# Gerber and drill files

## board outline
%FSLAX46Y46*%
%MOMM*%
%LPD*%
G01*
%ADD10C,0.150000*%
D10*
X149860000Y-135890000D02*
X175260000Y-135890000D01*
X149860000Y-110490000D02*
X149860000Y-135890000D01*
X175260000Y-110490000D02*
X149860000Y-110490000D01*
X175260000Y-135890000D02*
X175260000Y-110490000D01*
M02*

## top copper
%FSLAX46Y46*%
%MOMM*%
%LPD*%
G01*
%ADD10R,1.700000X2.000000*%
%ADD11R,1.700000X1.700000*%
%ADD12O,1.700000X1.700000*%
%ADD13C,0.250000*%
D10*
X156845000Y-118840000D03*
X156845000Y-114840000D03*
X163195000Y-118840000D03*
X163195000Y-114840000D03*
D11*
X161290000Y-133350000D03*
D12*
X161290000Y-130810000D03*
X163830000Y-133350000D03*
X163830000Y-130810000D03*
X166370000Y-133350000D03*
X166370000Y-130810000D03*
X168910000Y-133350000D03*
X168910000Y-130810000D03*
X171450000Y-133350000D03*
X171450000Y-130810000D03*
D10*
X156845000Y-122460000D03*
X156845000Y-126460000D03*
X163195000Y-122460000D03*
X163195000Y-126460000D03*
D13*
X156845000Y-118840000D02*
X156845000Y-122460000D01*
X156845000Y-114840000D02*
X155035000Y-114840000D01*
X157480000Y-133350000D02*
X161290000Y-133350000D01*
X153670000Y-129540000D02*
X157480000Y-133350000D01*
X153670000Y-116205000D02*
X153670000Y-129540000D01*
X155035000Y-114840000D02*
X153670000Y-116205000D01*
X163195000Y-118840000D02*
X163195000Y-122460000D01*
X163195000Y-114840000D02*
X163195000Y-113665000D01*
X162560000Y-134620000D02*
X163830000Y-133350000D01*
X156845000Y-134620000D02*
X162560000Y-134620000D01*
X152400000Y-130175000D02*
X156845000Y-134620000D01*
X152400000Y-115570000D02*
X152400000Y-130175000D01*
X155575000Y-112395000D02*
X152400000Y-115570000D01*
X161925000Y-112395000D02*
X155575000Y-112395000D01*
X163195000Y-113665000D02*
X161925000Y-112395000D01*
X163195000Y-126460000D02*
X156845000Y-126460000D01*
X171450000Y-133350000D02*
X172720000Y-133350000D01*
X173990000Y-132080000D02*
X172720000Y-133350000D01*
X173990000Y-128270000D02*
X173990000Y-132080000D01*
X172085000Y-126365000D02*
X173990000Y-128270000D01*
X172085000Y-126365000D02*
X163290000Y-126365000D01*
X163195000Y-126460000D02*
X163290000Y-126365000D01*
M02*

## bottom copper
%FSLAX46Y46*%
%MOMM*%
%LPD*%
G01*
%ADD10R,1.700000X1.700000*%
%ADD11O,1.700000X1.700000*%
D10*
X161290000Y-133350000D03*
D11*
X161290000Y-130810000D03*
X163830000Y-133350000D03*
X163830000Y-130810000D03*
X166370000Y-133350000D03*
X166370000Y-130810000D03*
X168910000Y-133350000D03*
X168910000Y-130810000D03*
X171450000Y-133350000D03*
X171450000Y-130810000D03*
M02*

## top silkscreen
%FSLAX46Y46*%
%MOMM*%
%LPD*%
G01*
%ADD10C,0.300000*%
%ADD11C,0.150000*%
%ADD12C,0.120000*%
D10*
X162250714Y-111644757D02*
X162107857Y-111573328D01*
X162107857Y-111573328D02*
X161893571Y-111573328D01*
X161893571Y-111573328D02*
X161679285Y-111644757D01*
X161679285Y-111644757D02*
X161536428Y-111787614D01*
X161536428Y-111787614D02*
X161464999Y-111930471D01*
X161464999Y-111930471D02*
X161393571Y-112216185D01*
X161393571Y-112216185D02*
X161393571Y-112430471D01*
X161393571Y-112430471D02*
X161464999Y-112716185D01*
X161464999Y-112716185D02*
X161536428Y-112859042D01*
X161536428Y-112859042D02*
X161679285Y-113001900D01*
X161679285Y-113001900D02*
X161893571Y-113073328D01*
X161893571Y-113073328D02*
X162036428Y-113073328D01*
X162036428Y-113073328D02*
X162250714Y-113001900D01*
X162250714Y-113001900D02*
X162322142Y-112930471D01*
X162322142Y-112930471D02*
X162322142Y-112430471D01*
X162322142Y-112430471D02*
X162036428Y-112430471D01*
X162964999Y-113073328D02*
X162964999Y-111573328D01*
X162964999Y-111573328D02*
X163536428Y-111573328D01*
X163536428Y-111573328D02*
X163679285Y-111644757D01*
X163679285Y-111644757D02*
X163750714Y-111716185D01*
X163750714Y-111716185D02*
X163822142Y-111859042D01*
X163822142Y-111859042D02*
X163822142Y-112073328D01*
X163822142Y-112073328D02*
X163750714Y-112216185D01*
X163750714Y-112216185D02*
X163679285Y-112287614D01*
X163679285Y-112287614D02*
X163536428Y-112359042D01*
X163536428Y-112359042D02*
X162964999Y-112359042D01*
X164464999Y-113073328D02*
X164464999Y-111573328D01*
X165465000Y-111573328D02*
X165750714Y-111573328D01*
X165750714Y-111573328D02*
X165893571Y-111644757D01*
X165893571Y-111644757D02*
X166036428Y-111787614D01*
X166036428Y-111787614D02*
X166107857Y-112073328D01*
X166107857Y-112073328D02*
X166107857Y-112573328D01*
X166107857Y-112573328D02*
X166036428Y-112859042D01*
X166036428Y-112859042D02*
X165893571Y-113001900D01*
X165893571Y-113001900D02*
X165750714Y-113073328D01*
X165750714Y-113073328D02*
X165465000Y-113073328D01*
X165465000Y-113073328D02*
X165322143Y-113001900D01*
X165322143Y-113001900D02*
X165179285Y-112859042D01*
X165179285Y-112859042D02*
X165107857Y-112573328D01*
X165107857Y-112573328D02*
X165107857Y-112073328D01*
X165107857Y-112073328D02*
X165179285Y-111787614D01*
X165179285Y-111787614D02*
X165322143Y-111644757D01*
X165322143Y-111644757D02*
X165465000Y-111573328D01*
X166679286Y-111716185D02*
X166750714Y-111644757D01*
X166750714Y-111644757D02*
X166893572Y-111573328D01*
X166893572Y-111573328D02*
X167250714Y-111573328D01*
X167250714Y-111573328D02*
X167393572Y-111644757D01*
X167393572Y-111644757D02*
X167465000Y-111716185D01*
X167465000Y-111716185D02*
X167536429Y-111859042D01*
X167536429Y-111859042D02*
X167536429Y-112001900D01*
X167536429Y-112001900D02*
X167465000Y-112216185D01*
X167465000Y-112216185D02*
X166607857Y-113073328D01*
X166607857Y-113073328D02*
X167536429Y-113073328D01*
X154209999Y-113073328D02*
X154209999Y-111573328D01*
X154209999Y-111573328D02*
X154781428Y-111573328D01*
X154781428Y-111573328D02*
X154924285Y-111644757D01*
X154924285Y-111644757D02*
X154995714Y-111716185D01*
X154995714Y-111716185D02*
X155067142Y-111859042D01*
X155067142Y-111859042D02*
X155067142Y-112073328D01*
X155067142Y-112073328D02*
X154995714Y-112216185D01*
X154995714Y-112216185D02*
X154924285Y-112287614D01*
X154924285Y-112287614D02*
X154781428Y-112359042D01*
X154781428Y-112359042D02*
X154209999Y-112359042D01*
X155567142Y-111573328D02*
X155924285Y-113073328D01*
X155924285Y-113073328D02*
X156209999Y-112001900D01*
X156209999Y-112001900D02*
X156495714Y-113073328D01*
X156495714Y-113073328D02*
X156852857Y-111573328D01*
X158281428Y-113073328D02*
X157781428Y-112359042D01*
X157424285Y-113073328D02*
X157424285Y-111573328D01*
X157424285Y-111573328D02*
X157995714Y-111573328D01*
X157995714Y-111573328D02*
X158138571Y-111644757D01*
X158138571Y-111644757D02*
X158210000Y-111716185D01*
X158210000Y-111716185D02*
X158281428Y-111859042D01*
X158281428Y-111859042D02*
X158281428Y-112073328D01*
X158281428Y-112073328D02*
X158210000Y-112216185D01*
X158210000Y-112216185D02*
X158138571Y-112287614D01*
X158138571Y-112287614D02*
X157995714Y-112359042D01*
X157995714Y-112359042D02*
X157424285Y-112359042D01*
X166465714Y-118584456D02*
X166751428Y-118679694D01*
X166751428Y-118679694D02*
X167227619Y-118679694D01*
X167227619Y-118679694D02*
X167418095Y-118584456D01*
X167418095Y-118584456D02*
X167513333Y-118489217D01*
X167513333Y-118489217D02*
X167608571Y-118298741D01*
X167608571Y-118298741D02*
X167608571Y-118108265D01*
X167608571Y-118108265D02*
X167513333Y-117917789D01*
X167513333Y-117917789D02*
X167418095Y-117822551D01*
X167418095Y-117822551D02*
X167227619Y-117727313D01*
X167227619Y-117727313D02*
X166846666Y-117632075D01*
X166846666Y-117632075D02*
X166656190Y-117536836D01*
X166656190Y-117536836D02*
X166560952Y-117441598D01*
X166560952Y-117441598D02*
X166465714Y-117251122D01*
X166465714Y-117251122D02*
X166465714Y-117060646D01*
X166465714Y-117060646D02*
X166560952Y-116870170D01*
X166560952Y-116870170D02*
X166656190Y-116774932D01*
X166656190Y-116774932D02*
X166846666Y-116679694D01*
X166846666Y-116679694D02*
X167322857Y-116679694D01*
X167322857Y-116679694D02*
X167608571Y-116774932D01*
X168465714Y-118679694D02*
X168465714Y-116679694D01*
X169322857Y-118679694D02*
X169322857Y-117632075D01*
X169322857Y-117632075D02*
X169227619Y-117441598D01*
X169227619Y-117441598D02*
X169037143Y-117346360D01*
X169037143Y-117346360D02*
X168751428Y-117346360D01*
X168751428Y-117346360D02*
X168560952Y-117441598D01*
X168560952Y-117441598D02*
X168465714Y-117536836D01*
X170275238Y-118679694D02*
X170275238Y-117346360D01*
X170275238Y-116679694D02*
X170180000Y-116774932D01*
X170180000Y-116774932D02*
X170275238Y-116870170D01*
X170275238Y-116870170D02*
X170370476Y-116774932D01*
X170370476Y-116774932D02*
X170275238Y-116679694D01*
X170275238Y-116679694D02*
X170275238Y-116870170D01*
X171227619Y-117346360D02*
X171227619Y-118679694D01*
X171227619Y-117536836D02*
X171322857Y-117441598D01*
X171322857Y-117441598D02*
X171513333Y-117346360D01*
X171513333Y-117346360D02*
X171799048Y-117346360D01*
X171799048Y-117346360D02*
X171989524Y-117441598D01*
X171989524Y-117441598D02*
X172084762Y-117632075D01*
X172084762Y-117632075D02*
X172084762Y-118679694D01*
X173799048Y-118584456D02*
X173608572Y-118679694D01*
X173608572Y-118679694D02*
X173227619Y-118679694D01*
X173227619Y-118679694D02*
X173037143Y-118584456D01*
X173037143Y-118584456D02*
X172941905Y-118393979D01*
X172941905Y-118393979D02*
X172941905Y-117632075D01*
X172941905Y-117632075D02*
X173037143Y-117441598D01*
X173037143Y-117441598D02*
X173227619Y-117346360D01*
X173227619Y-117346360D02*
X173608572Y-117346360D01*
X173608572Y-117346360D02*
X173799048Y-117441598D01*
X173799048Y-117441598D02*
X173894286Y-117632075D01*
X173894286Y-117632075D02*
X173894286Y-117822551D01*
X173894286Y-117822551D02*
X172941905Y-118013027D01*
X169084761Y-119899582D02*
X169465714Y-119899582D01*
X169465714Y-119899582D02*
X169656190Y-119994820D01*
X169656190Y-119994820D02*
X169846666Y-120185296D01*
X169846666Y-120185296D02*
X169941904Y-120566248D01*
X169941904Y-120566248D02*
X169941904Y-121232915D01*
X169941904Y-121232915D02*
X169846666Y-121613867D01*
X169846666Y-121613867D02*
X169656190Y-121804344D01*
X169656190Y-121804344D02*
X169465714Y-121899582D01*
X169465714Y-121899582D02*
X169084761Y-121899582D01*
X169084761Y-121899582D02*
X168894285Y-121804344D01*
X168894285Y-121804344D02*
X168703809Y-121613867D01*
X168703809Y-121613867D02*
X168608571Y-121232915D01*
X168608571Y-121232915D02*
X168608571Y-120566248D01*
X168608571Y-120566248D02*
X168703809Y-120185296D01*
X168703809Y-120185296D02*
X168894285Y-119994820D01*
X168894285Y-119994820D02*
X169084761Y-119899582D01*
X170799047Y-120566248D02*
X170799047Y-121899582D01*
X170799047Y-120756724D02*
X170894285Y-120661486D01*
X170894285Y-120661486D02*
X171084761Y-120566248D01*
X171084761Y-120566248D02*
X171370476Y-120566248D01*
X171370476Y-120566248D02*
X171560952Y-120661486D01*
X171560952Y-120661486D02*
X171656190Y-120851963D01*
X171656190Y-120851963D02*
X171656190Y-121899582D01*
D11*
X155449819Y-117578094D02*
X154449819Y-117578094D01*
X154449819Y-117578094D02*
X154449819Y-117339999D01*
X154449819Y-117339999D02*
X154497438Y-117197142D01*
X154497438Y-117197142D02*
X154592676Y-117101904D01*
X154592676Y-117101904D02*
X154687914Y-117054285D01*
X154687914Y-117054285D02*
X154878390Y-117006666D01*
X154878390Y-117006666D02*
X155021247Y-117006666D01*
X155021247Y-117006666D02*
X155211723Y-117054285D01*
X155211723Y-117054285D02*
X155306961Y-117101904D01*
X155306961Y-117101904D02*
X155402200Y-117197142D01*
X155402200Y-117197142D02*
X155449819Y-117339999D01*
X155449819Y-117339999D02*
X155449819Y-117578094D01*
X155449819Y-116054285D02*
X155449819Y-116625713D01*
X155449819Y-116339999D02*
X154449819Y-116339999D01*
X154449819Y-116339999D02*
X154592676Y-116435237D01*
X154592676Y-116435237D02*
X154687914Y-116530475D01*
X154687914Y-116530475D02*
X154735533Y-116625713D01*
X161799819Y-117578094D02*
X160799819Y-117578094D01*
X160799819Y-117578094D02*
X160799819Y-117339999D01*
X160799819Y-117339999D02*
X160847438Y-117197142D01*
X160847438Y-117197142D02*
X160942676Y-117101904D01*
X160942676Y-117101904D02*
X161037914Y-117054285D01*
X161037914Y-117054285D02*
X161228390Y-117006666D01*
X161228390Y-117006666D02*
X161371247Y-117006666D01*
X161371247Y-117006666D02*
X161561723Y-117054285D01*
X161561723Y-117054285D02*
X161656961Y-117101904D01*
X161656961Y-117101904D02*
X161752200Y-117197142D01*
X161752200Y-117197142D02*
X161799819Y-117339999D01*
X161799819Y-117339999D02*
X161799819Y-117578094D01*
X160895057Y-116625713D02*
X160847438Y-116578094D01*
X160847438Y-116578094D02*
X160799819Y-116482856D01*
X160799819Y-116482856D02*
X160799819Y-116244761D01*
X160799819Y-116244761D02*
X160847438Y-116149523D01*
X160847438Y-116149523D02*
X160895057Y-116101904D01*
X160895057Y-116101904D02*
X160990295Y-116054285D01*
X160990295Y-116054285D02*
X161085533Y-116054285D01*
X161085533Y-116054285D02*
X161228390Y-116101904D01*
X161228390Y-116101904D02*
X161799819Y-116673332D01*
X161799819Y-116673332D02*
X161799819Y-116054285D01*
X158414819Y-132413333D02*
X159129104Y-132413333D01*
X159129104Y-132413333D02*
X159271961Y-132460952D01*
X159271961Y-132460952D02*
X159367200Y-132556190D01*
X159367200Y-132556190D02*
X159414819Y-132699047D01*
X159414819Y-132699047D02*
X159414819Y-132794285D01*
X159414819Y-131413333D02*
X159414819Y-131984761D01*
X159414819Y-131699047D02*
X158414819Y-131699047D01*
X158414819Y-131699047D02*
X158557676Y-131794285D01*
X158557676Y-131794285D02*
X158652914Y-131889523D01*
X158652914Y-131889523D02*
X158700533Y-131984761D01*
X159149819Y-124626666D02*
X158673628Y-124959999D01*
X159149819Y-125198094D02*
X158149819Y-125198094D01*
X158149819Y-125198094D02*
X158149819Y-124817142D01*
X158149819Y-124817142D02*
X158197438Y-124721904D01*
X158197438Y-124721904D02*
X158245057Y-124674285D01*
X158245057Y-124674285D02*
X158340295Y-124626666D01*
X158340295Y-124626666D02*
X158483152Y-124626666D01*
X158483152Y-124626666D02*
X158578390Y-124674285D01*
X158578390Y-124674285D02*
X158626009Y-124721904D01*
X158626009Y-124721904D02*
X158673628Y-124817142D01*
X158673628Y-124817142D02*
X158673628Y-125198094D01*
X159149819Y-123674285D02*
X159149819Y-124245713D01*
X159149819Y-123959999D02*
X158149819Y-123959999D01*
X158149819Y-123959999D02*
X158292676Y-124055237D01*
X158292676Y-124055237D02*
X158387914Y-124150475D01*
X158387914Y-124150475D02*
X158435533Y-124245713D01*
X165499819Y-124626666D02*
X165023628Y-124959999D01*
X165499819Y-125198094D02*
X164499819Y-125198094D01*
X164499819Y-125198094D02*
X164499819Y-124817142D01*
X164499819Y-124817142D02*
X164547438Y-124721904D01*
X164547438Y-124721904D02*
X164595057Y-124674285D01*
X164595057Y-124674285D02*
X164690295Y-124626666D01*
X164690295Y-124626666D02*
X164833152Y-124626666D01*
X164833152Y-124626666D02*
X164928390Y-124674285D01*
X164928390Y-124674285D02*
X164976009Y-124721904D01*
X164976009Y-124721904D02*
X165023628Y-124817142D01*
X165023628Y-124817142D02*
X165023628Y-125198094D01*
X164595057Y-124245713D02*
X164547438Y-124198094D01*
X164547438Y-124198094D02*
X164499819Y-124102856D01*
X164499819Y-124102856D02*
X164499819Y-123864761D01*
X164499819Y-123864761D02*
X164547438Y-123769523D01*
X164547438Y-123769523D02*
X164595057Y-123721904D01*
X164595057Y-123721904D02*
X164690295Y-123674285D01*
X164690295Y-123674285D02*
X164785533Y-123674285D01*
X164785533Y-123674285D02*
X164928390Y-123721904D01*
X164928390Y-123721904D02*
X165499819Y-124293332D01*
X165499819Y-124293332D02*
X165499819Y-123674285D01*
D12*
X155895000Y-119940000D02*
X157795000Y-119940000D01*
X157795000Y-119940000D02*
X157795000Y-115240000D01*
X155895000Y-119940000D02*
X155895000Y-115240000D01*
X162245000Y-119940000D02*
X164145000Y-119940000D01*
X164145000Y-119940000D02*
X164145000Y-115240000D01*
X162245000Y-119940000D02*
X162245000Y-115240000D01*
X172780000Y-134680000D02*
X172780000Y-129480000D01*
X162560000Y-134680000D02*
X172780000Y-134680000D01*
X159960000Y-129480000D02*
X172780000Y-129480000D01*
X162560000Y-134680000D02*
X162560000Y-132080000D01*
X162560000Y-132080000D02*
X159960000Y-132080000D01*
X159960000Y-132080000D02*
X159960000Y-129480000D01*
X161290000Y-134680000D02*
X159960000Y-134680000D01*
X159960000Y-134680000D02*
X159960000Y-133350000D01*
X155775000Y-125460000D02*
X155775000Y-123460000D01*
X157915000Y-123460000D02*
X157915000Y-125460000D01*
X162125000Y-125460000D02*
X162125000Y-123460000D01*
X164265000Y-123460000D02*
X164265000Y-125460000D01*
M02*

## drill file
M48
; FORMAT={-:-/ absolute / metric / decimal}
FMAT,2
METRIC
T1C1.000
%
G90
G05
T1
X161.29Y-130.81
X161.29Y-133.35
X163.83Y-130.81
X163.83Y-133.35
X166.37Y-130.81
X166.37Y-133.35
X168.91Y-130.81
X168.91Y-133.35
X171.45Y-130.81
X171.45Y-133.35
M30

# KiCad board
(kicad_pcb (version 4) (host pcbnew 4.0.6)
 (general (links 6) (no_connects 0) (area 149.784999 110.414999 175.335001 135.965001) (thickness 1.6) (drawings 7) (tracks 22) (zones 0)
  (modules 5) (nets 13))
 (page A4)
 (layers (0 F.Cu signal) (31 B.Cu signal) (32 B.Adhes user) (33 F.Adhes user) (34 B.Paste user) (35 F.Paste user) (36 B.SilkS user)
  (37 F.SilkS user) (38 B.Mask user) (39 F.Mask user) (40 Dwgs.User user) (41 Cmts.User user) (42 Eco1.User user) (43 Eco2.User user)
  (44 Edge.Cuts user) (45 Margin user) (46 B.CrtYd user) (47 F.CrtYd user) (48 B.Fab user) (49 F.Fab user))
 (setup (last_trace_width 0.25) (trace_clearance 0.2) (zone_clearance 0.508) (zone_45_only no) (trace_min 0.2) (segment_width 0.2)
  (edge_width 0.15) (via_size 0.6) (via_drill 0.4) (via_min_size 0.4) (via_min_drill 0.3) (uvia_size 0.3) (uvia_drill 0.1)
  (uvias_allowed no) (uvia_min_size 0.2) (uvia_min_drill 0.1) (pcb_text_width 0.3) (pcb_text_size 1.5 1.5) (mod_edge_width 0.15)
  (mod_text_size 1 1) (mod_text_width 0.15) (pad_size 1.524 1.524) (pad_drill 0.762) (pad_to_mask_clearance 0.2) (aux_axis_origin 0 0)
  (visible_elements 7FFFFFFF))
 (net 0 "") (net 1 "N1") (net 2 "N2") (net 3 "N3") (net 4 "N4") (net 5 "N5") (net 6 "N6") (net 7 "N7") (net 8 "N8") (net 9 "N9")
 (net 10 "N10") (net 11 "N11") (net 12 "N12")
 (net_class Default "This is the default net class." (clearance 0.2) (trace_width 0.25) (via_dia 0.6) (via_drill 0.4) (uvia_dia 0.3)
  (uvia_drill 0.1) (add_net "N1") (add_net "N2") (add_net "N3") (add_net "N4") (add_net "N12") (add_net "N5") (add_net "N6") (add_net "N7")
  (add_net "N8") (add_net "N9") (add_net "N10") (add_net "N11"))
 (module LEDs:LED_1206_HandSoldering (layer F.Cu) (at 156.845 116.84 90)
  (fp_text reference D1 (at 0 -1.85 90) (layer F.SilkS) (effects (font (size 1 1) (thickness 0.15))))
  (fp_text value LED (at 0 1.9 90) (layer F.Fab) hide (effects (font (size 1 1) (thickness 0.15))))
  (fp_line (start -3.1 -0.95) (end -3.1 0.95) (layer F.SilkS) (width 0.12))
  (fp_line (start -3.1 0.95) (end 1.6 0.95) (layer F.SilkS) (width 0.12))
  (fp_line (start -3.1 -0.95) (end 1.6 -0.95) (layer F.SilkS) (width 0.12))
  (pad 1 smd rect (at -2 0 90) (size 2 1.7) (layers F.Cu F.Paste F.Mask) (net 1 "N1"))
  (pad 2 smd rect (at 2 0 90) (size 2 1.7) (layers F.Cu F.Paste F.Mask) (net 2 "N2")))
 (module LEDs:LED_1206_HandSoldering (layer F.Cu) (at 163.195 116.84 90)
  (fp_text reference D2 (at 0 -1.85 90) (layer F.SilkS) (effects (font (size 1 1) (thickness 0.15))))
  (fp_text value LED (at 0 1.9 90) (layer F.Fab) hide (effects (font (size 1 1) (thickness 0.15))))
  (fp_line (start -3.1 -0.95) (end -3.1 0.95) (layer F.SilkS) (width 0.12))
  (fp_line (start -3.1 0.95) (end 1.6 0.95) (layer F.SilkS) (width 0.12))
  (fp_line (start -3.1 -0.95) (end 1.6 -0.95) (layer F.SilkS) (width 0.12))
  (pad 1 smd rect (at -2 0 90) (size 2 1.7) (layers F.Cu F.Paste F.Mask) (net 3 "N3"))
  (pad 2 smd rect (at 2 0 90) (size 2 1.7) (layers F.Cu F.Paste F.Mask) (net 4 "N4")))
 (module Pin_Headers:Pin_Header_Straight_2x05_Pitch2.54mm (layer F.Cu) (at 161.29 133.35 90)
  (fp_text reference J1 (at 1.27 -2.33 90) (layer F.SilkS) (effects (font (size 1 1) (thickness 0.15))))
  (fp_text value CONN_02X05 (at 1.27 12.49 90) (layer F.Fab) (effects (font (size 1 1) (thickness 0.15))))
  (fp_line (start -1.33 11.49) (end 3.87 11.49) (layer F.SilkS) (width 0.12))
  (fp_line (start -1.33 1.27) (end -1.33 11.49) (layer F.SilkS) (width 0.12))
  (fp_line (start 3.87 -1.33) (end 3.87 11.49) (layer F.SilkS) (width 0.12))
  (fp_line (start -1.33 1.27) (end 1.27 1.27) (layer F.SilkS) (width 0.12))
  (fp_line (start 1.27 1.27) (end 1.27 -1.33) (layer F.SilkS) (width 0.12))
  (fp_line (start 1.27 -1.33) (end 3.87 -1.33) (layer F.SilkS) (width 0.12))
  (fp_line (start -1.33 0) (end -1.33 -1.33) (layer F.SilkS) (width 0.12))
  (fp_line (start -1.33 -1.33) (end 0 -1.33) (layer F.SilkS) (width 0.12))
  (pad 1 thru_hole rect (at 0 0 90) (size 1.7 1.7) (drill 1) (layers *.Cu *.Mask) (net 2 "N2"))
  (pad 2 thru_hole oval (at 2.54 0 90) (size 1.7 1.7) (drill 1) (layers *.Cu *.Mask) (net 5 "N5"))
  (pad 3 thru_hole oval (at 0 2.54 90) (size 1.7 1.7) (drill 1) (layers *.Cu *.Mask) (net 4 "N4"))
  (pad 4 thru_hole oval (at 2.54 2.54 90) (size 1.7 1.7) (drill 1) (layers *.Cu *.Mask) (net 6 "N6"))
  (pad 5 thru_hole oval (at 0 5.08 90) (size 1.7 1.7) (drill 1) (layers *.Cu *.Mask) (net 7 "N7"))
  (pad 6 thru_hole oval (at 2.54 5.08 90) (size 1.7 1.7) (drill 1) (layers *.Cu *.Mask) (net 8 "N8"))
  (pad 7 thru_hole oval (at 0 7.62 90) (size 1.7 1.7) (drill 1) (layers *.Cu *.Mask) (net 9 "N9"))
  (pad 8 thru_hole oval (at 2.54 7.62 90) (size 1.7 1.7) (drill 1) (layers *.Cu *.Mask) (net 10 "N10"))
  (pad 9 thru_hole oval (at 0 10.16 90) (size 1.7 1.7) (drill 1) (layers *.Cu *.Mask) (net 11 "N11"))
  (pad 10 thru_hole oval (at 2.54 10.16 90) (size 1.7 1.7) (drill 1) (layers *.Cu *.Mask) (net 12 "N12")))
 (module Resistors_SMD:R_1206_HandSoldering (layer F.Cu) (at 156.845 124.46 270)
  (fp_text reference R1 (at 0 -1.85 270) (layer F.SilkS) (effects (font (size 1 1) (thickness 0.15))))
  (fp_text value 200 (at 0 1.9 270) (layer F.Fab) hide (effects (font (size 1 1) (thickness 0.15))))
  (fp_line (start 1 1.07) (end -1 1.07) (layer F.SilkS) (width 0.12))
  (fp_line (start -1 -1.07) (end 1 -1.07) (layer F.SilkS) (width 0.12))
  (pad 1 smd rect (at -2 0 270) (size 2 1.7) (layers F.Cu F.Paste F.Mask) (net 1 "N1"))
  (pad 2 smd rect (at 2 0 270) (size 2 1.7) (layers F.Cu F.Paste F.Mask) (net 11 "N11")))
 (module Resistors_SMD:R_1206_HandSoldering (layer F.Cu) (at 163.195 124.46 270)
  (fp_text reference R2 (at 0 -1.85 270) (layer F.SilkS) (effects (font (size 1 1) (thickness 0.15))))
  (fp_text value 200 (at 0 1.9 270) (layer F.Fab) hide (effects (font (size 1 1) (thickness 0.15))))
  (fp_line (start 1 1.07) (end -1 1.07) (layer F.SilkS) (width 0.12))
  (fp_line (start -1 -1.07) (end 1 -1.07) (layer F.SilkS) (width 0.12))
  (pad 1 smd rect (at -2 0 270) (size 2 1.7) (layers F.Cu F.Paste F.Mask) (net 3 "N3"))
  (pad 2 smd rect (at 2 0 270) (size 2 1.7) (layers F.Cu F.Paste F.Mask) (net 11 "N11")))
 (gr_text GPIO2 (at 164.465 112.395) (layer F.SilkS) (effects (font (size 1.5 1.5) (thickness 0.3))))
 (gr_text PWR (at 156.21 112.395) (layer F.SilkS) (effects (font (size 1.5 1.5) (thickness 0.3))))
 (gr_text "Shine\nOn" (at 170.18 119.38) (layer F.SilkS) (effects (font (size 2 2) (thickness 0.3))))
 (gr_line (start 149.86 135.89) (end 175.26 135.89) (angle 90) (layer Edge.Cuts) (width 0.15))
 (gr_line (start 149.86 110.49) (end 149.86 135.89) (angle 90) (layer Edge.Cuts) (width 0.15))
 (gr_line (start 175.26 110.49) (end 149.86 110.49) (angle 90) (layer Edge.Cuts) (width 0.15))
 (gr_line (start 175.26 135.89) (end 175.26 110.49) (angle 90) (layer Edge.Cuts) (width 0.15))
 (segment (start 156.845 118.84) (end 156.845 122.46) (width 0.25) (layer F.Cu) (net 1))
 (segment (start 156.845 114.84) (end 155.035 114.84) (width 0.25) (layer F.Cu) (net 2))
 (segment (start 157.48 133.35) (end 161.29 133.35) (width 0.25) (layer F.Cu) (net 2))
 (segment (start 153.67 129.54) (end 157.48 133.35) (width 0.25) (layer F.Cu) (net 2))
 (segment (start 153.67 116.205) (end 153.67 129.54) (width 0.25) (layer F.Cu) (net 2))
 (segment (start 155.035 114.84) (end 153.67 116.205) (width 0.25) (layer F.Cu) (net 2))
 (segment (start 163.195 118.84) (end 163.195 122.46) (width 0.25) (layer F.Cu) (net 3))
 (segment (start 163.195 114.84) (end 163.195 113.665) (width 0.25) (layer F.Cu) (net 4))
 (segment (start 162.56 134.62) (end 163.83 133.35) (width 0.25) (layer F.Cu) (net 4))
 (segment (start 156.845 134.62) (end 162.56 134.62) (width 0.25) (layer F.Cu) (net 4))
 (segment (start 152.4 130.175) (end 156.845 134.62) (width 0.25) (layer F.Cu) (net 4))
 (segment (start 152.4 115.57) (end 152.4 130.175) (width 0.25) (layer F.Cu) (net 4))
 (segment (start 155.575 112.395) (end 152.4 115.57) (width 0.25) (layer F.Cu) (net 4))
 (segment (start 161.925 112.395) (end 155.575 112.395) (width 0.25) (layer F.Cu) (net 4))
 (segment (start 163.195 113.665) (end 161.925 112.395) (width 0.25) (layer F.Cu) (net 4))
 (segment (start 163.195 126.46) (end 156.845 126.46) (width 0.25) (layer F.Cu) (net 11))
 (segment (start 171.45 133.35) (end 172.72 133.35) (width 0.25) (layer F.Cu) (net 11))
 (segment (start 173.99 132.08) (end 172.72 133.35) (width 0.25) (layer F.Cu) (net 11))
 (segment (start 173.99 128.27) (end 173.99 132.08) (width 0.25) (layer F.Cu) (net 11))
 (segment (start 172.085 126.365) (end 173.99 128.27) (width 0.25) (layer F.Cu) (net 11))
 (segment (start 172.085 126.365) (end 163.29 126.365) (width 0.25) (layer F.Cu) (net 11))
 (segment (start 163.195 126.46) (end 163.29 126.365) (width 0.25) (layer F.Cu) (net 11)))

